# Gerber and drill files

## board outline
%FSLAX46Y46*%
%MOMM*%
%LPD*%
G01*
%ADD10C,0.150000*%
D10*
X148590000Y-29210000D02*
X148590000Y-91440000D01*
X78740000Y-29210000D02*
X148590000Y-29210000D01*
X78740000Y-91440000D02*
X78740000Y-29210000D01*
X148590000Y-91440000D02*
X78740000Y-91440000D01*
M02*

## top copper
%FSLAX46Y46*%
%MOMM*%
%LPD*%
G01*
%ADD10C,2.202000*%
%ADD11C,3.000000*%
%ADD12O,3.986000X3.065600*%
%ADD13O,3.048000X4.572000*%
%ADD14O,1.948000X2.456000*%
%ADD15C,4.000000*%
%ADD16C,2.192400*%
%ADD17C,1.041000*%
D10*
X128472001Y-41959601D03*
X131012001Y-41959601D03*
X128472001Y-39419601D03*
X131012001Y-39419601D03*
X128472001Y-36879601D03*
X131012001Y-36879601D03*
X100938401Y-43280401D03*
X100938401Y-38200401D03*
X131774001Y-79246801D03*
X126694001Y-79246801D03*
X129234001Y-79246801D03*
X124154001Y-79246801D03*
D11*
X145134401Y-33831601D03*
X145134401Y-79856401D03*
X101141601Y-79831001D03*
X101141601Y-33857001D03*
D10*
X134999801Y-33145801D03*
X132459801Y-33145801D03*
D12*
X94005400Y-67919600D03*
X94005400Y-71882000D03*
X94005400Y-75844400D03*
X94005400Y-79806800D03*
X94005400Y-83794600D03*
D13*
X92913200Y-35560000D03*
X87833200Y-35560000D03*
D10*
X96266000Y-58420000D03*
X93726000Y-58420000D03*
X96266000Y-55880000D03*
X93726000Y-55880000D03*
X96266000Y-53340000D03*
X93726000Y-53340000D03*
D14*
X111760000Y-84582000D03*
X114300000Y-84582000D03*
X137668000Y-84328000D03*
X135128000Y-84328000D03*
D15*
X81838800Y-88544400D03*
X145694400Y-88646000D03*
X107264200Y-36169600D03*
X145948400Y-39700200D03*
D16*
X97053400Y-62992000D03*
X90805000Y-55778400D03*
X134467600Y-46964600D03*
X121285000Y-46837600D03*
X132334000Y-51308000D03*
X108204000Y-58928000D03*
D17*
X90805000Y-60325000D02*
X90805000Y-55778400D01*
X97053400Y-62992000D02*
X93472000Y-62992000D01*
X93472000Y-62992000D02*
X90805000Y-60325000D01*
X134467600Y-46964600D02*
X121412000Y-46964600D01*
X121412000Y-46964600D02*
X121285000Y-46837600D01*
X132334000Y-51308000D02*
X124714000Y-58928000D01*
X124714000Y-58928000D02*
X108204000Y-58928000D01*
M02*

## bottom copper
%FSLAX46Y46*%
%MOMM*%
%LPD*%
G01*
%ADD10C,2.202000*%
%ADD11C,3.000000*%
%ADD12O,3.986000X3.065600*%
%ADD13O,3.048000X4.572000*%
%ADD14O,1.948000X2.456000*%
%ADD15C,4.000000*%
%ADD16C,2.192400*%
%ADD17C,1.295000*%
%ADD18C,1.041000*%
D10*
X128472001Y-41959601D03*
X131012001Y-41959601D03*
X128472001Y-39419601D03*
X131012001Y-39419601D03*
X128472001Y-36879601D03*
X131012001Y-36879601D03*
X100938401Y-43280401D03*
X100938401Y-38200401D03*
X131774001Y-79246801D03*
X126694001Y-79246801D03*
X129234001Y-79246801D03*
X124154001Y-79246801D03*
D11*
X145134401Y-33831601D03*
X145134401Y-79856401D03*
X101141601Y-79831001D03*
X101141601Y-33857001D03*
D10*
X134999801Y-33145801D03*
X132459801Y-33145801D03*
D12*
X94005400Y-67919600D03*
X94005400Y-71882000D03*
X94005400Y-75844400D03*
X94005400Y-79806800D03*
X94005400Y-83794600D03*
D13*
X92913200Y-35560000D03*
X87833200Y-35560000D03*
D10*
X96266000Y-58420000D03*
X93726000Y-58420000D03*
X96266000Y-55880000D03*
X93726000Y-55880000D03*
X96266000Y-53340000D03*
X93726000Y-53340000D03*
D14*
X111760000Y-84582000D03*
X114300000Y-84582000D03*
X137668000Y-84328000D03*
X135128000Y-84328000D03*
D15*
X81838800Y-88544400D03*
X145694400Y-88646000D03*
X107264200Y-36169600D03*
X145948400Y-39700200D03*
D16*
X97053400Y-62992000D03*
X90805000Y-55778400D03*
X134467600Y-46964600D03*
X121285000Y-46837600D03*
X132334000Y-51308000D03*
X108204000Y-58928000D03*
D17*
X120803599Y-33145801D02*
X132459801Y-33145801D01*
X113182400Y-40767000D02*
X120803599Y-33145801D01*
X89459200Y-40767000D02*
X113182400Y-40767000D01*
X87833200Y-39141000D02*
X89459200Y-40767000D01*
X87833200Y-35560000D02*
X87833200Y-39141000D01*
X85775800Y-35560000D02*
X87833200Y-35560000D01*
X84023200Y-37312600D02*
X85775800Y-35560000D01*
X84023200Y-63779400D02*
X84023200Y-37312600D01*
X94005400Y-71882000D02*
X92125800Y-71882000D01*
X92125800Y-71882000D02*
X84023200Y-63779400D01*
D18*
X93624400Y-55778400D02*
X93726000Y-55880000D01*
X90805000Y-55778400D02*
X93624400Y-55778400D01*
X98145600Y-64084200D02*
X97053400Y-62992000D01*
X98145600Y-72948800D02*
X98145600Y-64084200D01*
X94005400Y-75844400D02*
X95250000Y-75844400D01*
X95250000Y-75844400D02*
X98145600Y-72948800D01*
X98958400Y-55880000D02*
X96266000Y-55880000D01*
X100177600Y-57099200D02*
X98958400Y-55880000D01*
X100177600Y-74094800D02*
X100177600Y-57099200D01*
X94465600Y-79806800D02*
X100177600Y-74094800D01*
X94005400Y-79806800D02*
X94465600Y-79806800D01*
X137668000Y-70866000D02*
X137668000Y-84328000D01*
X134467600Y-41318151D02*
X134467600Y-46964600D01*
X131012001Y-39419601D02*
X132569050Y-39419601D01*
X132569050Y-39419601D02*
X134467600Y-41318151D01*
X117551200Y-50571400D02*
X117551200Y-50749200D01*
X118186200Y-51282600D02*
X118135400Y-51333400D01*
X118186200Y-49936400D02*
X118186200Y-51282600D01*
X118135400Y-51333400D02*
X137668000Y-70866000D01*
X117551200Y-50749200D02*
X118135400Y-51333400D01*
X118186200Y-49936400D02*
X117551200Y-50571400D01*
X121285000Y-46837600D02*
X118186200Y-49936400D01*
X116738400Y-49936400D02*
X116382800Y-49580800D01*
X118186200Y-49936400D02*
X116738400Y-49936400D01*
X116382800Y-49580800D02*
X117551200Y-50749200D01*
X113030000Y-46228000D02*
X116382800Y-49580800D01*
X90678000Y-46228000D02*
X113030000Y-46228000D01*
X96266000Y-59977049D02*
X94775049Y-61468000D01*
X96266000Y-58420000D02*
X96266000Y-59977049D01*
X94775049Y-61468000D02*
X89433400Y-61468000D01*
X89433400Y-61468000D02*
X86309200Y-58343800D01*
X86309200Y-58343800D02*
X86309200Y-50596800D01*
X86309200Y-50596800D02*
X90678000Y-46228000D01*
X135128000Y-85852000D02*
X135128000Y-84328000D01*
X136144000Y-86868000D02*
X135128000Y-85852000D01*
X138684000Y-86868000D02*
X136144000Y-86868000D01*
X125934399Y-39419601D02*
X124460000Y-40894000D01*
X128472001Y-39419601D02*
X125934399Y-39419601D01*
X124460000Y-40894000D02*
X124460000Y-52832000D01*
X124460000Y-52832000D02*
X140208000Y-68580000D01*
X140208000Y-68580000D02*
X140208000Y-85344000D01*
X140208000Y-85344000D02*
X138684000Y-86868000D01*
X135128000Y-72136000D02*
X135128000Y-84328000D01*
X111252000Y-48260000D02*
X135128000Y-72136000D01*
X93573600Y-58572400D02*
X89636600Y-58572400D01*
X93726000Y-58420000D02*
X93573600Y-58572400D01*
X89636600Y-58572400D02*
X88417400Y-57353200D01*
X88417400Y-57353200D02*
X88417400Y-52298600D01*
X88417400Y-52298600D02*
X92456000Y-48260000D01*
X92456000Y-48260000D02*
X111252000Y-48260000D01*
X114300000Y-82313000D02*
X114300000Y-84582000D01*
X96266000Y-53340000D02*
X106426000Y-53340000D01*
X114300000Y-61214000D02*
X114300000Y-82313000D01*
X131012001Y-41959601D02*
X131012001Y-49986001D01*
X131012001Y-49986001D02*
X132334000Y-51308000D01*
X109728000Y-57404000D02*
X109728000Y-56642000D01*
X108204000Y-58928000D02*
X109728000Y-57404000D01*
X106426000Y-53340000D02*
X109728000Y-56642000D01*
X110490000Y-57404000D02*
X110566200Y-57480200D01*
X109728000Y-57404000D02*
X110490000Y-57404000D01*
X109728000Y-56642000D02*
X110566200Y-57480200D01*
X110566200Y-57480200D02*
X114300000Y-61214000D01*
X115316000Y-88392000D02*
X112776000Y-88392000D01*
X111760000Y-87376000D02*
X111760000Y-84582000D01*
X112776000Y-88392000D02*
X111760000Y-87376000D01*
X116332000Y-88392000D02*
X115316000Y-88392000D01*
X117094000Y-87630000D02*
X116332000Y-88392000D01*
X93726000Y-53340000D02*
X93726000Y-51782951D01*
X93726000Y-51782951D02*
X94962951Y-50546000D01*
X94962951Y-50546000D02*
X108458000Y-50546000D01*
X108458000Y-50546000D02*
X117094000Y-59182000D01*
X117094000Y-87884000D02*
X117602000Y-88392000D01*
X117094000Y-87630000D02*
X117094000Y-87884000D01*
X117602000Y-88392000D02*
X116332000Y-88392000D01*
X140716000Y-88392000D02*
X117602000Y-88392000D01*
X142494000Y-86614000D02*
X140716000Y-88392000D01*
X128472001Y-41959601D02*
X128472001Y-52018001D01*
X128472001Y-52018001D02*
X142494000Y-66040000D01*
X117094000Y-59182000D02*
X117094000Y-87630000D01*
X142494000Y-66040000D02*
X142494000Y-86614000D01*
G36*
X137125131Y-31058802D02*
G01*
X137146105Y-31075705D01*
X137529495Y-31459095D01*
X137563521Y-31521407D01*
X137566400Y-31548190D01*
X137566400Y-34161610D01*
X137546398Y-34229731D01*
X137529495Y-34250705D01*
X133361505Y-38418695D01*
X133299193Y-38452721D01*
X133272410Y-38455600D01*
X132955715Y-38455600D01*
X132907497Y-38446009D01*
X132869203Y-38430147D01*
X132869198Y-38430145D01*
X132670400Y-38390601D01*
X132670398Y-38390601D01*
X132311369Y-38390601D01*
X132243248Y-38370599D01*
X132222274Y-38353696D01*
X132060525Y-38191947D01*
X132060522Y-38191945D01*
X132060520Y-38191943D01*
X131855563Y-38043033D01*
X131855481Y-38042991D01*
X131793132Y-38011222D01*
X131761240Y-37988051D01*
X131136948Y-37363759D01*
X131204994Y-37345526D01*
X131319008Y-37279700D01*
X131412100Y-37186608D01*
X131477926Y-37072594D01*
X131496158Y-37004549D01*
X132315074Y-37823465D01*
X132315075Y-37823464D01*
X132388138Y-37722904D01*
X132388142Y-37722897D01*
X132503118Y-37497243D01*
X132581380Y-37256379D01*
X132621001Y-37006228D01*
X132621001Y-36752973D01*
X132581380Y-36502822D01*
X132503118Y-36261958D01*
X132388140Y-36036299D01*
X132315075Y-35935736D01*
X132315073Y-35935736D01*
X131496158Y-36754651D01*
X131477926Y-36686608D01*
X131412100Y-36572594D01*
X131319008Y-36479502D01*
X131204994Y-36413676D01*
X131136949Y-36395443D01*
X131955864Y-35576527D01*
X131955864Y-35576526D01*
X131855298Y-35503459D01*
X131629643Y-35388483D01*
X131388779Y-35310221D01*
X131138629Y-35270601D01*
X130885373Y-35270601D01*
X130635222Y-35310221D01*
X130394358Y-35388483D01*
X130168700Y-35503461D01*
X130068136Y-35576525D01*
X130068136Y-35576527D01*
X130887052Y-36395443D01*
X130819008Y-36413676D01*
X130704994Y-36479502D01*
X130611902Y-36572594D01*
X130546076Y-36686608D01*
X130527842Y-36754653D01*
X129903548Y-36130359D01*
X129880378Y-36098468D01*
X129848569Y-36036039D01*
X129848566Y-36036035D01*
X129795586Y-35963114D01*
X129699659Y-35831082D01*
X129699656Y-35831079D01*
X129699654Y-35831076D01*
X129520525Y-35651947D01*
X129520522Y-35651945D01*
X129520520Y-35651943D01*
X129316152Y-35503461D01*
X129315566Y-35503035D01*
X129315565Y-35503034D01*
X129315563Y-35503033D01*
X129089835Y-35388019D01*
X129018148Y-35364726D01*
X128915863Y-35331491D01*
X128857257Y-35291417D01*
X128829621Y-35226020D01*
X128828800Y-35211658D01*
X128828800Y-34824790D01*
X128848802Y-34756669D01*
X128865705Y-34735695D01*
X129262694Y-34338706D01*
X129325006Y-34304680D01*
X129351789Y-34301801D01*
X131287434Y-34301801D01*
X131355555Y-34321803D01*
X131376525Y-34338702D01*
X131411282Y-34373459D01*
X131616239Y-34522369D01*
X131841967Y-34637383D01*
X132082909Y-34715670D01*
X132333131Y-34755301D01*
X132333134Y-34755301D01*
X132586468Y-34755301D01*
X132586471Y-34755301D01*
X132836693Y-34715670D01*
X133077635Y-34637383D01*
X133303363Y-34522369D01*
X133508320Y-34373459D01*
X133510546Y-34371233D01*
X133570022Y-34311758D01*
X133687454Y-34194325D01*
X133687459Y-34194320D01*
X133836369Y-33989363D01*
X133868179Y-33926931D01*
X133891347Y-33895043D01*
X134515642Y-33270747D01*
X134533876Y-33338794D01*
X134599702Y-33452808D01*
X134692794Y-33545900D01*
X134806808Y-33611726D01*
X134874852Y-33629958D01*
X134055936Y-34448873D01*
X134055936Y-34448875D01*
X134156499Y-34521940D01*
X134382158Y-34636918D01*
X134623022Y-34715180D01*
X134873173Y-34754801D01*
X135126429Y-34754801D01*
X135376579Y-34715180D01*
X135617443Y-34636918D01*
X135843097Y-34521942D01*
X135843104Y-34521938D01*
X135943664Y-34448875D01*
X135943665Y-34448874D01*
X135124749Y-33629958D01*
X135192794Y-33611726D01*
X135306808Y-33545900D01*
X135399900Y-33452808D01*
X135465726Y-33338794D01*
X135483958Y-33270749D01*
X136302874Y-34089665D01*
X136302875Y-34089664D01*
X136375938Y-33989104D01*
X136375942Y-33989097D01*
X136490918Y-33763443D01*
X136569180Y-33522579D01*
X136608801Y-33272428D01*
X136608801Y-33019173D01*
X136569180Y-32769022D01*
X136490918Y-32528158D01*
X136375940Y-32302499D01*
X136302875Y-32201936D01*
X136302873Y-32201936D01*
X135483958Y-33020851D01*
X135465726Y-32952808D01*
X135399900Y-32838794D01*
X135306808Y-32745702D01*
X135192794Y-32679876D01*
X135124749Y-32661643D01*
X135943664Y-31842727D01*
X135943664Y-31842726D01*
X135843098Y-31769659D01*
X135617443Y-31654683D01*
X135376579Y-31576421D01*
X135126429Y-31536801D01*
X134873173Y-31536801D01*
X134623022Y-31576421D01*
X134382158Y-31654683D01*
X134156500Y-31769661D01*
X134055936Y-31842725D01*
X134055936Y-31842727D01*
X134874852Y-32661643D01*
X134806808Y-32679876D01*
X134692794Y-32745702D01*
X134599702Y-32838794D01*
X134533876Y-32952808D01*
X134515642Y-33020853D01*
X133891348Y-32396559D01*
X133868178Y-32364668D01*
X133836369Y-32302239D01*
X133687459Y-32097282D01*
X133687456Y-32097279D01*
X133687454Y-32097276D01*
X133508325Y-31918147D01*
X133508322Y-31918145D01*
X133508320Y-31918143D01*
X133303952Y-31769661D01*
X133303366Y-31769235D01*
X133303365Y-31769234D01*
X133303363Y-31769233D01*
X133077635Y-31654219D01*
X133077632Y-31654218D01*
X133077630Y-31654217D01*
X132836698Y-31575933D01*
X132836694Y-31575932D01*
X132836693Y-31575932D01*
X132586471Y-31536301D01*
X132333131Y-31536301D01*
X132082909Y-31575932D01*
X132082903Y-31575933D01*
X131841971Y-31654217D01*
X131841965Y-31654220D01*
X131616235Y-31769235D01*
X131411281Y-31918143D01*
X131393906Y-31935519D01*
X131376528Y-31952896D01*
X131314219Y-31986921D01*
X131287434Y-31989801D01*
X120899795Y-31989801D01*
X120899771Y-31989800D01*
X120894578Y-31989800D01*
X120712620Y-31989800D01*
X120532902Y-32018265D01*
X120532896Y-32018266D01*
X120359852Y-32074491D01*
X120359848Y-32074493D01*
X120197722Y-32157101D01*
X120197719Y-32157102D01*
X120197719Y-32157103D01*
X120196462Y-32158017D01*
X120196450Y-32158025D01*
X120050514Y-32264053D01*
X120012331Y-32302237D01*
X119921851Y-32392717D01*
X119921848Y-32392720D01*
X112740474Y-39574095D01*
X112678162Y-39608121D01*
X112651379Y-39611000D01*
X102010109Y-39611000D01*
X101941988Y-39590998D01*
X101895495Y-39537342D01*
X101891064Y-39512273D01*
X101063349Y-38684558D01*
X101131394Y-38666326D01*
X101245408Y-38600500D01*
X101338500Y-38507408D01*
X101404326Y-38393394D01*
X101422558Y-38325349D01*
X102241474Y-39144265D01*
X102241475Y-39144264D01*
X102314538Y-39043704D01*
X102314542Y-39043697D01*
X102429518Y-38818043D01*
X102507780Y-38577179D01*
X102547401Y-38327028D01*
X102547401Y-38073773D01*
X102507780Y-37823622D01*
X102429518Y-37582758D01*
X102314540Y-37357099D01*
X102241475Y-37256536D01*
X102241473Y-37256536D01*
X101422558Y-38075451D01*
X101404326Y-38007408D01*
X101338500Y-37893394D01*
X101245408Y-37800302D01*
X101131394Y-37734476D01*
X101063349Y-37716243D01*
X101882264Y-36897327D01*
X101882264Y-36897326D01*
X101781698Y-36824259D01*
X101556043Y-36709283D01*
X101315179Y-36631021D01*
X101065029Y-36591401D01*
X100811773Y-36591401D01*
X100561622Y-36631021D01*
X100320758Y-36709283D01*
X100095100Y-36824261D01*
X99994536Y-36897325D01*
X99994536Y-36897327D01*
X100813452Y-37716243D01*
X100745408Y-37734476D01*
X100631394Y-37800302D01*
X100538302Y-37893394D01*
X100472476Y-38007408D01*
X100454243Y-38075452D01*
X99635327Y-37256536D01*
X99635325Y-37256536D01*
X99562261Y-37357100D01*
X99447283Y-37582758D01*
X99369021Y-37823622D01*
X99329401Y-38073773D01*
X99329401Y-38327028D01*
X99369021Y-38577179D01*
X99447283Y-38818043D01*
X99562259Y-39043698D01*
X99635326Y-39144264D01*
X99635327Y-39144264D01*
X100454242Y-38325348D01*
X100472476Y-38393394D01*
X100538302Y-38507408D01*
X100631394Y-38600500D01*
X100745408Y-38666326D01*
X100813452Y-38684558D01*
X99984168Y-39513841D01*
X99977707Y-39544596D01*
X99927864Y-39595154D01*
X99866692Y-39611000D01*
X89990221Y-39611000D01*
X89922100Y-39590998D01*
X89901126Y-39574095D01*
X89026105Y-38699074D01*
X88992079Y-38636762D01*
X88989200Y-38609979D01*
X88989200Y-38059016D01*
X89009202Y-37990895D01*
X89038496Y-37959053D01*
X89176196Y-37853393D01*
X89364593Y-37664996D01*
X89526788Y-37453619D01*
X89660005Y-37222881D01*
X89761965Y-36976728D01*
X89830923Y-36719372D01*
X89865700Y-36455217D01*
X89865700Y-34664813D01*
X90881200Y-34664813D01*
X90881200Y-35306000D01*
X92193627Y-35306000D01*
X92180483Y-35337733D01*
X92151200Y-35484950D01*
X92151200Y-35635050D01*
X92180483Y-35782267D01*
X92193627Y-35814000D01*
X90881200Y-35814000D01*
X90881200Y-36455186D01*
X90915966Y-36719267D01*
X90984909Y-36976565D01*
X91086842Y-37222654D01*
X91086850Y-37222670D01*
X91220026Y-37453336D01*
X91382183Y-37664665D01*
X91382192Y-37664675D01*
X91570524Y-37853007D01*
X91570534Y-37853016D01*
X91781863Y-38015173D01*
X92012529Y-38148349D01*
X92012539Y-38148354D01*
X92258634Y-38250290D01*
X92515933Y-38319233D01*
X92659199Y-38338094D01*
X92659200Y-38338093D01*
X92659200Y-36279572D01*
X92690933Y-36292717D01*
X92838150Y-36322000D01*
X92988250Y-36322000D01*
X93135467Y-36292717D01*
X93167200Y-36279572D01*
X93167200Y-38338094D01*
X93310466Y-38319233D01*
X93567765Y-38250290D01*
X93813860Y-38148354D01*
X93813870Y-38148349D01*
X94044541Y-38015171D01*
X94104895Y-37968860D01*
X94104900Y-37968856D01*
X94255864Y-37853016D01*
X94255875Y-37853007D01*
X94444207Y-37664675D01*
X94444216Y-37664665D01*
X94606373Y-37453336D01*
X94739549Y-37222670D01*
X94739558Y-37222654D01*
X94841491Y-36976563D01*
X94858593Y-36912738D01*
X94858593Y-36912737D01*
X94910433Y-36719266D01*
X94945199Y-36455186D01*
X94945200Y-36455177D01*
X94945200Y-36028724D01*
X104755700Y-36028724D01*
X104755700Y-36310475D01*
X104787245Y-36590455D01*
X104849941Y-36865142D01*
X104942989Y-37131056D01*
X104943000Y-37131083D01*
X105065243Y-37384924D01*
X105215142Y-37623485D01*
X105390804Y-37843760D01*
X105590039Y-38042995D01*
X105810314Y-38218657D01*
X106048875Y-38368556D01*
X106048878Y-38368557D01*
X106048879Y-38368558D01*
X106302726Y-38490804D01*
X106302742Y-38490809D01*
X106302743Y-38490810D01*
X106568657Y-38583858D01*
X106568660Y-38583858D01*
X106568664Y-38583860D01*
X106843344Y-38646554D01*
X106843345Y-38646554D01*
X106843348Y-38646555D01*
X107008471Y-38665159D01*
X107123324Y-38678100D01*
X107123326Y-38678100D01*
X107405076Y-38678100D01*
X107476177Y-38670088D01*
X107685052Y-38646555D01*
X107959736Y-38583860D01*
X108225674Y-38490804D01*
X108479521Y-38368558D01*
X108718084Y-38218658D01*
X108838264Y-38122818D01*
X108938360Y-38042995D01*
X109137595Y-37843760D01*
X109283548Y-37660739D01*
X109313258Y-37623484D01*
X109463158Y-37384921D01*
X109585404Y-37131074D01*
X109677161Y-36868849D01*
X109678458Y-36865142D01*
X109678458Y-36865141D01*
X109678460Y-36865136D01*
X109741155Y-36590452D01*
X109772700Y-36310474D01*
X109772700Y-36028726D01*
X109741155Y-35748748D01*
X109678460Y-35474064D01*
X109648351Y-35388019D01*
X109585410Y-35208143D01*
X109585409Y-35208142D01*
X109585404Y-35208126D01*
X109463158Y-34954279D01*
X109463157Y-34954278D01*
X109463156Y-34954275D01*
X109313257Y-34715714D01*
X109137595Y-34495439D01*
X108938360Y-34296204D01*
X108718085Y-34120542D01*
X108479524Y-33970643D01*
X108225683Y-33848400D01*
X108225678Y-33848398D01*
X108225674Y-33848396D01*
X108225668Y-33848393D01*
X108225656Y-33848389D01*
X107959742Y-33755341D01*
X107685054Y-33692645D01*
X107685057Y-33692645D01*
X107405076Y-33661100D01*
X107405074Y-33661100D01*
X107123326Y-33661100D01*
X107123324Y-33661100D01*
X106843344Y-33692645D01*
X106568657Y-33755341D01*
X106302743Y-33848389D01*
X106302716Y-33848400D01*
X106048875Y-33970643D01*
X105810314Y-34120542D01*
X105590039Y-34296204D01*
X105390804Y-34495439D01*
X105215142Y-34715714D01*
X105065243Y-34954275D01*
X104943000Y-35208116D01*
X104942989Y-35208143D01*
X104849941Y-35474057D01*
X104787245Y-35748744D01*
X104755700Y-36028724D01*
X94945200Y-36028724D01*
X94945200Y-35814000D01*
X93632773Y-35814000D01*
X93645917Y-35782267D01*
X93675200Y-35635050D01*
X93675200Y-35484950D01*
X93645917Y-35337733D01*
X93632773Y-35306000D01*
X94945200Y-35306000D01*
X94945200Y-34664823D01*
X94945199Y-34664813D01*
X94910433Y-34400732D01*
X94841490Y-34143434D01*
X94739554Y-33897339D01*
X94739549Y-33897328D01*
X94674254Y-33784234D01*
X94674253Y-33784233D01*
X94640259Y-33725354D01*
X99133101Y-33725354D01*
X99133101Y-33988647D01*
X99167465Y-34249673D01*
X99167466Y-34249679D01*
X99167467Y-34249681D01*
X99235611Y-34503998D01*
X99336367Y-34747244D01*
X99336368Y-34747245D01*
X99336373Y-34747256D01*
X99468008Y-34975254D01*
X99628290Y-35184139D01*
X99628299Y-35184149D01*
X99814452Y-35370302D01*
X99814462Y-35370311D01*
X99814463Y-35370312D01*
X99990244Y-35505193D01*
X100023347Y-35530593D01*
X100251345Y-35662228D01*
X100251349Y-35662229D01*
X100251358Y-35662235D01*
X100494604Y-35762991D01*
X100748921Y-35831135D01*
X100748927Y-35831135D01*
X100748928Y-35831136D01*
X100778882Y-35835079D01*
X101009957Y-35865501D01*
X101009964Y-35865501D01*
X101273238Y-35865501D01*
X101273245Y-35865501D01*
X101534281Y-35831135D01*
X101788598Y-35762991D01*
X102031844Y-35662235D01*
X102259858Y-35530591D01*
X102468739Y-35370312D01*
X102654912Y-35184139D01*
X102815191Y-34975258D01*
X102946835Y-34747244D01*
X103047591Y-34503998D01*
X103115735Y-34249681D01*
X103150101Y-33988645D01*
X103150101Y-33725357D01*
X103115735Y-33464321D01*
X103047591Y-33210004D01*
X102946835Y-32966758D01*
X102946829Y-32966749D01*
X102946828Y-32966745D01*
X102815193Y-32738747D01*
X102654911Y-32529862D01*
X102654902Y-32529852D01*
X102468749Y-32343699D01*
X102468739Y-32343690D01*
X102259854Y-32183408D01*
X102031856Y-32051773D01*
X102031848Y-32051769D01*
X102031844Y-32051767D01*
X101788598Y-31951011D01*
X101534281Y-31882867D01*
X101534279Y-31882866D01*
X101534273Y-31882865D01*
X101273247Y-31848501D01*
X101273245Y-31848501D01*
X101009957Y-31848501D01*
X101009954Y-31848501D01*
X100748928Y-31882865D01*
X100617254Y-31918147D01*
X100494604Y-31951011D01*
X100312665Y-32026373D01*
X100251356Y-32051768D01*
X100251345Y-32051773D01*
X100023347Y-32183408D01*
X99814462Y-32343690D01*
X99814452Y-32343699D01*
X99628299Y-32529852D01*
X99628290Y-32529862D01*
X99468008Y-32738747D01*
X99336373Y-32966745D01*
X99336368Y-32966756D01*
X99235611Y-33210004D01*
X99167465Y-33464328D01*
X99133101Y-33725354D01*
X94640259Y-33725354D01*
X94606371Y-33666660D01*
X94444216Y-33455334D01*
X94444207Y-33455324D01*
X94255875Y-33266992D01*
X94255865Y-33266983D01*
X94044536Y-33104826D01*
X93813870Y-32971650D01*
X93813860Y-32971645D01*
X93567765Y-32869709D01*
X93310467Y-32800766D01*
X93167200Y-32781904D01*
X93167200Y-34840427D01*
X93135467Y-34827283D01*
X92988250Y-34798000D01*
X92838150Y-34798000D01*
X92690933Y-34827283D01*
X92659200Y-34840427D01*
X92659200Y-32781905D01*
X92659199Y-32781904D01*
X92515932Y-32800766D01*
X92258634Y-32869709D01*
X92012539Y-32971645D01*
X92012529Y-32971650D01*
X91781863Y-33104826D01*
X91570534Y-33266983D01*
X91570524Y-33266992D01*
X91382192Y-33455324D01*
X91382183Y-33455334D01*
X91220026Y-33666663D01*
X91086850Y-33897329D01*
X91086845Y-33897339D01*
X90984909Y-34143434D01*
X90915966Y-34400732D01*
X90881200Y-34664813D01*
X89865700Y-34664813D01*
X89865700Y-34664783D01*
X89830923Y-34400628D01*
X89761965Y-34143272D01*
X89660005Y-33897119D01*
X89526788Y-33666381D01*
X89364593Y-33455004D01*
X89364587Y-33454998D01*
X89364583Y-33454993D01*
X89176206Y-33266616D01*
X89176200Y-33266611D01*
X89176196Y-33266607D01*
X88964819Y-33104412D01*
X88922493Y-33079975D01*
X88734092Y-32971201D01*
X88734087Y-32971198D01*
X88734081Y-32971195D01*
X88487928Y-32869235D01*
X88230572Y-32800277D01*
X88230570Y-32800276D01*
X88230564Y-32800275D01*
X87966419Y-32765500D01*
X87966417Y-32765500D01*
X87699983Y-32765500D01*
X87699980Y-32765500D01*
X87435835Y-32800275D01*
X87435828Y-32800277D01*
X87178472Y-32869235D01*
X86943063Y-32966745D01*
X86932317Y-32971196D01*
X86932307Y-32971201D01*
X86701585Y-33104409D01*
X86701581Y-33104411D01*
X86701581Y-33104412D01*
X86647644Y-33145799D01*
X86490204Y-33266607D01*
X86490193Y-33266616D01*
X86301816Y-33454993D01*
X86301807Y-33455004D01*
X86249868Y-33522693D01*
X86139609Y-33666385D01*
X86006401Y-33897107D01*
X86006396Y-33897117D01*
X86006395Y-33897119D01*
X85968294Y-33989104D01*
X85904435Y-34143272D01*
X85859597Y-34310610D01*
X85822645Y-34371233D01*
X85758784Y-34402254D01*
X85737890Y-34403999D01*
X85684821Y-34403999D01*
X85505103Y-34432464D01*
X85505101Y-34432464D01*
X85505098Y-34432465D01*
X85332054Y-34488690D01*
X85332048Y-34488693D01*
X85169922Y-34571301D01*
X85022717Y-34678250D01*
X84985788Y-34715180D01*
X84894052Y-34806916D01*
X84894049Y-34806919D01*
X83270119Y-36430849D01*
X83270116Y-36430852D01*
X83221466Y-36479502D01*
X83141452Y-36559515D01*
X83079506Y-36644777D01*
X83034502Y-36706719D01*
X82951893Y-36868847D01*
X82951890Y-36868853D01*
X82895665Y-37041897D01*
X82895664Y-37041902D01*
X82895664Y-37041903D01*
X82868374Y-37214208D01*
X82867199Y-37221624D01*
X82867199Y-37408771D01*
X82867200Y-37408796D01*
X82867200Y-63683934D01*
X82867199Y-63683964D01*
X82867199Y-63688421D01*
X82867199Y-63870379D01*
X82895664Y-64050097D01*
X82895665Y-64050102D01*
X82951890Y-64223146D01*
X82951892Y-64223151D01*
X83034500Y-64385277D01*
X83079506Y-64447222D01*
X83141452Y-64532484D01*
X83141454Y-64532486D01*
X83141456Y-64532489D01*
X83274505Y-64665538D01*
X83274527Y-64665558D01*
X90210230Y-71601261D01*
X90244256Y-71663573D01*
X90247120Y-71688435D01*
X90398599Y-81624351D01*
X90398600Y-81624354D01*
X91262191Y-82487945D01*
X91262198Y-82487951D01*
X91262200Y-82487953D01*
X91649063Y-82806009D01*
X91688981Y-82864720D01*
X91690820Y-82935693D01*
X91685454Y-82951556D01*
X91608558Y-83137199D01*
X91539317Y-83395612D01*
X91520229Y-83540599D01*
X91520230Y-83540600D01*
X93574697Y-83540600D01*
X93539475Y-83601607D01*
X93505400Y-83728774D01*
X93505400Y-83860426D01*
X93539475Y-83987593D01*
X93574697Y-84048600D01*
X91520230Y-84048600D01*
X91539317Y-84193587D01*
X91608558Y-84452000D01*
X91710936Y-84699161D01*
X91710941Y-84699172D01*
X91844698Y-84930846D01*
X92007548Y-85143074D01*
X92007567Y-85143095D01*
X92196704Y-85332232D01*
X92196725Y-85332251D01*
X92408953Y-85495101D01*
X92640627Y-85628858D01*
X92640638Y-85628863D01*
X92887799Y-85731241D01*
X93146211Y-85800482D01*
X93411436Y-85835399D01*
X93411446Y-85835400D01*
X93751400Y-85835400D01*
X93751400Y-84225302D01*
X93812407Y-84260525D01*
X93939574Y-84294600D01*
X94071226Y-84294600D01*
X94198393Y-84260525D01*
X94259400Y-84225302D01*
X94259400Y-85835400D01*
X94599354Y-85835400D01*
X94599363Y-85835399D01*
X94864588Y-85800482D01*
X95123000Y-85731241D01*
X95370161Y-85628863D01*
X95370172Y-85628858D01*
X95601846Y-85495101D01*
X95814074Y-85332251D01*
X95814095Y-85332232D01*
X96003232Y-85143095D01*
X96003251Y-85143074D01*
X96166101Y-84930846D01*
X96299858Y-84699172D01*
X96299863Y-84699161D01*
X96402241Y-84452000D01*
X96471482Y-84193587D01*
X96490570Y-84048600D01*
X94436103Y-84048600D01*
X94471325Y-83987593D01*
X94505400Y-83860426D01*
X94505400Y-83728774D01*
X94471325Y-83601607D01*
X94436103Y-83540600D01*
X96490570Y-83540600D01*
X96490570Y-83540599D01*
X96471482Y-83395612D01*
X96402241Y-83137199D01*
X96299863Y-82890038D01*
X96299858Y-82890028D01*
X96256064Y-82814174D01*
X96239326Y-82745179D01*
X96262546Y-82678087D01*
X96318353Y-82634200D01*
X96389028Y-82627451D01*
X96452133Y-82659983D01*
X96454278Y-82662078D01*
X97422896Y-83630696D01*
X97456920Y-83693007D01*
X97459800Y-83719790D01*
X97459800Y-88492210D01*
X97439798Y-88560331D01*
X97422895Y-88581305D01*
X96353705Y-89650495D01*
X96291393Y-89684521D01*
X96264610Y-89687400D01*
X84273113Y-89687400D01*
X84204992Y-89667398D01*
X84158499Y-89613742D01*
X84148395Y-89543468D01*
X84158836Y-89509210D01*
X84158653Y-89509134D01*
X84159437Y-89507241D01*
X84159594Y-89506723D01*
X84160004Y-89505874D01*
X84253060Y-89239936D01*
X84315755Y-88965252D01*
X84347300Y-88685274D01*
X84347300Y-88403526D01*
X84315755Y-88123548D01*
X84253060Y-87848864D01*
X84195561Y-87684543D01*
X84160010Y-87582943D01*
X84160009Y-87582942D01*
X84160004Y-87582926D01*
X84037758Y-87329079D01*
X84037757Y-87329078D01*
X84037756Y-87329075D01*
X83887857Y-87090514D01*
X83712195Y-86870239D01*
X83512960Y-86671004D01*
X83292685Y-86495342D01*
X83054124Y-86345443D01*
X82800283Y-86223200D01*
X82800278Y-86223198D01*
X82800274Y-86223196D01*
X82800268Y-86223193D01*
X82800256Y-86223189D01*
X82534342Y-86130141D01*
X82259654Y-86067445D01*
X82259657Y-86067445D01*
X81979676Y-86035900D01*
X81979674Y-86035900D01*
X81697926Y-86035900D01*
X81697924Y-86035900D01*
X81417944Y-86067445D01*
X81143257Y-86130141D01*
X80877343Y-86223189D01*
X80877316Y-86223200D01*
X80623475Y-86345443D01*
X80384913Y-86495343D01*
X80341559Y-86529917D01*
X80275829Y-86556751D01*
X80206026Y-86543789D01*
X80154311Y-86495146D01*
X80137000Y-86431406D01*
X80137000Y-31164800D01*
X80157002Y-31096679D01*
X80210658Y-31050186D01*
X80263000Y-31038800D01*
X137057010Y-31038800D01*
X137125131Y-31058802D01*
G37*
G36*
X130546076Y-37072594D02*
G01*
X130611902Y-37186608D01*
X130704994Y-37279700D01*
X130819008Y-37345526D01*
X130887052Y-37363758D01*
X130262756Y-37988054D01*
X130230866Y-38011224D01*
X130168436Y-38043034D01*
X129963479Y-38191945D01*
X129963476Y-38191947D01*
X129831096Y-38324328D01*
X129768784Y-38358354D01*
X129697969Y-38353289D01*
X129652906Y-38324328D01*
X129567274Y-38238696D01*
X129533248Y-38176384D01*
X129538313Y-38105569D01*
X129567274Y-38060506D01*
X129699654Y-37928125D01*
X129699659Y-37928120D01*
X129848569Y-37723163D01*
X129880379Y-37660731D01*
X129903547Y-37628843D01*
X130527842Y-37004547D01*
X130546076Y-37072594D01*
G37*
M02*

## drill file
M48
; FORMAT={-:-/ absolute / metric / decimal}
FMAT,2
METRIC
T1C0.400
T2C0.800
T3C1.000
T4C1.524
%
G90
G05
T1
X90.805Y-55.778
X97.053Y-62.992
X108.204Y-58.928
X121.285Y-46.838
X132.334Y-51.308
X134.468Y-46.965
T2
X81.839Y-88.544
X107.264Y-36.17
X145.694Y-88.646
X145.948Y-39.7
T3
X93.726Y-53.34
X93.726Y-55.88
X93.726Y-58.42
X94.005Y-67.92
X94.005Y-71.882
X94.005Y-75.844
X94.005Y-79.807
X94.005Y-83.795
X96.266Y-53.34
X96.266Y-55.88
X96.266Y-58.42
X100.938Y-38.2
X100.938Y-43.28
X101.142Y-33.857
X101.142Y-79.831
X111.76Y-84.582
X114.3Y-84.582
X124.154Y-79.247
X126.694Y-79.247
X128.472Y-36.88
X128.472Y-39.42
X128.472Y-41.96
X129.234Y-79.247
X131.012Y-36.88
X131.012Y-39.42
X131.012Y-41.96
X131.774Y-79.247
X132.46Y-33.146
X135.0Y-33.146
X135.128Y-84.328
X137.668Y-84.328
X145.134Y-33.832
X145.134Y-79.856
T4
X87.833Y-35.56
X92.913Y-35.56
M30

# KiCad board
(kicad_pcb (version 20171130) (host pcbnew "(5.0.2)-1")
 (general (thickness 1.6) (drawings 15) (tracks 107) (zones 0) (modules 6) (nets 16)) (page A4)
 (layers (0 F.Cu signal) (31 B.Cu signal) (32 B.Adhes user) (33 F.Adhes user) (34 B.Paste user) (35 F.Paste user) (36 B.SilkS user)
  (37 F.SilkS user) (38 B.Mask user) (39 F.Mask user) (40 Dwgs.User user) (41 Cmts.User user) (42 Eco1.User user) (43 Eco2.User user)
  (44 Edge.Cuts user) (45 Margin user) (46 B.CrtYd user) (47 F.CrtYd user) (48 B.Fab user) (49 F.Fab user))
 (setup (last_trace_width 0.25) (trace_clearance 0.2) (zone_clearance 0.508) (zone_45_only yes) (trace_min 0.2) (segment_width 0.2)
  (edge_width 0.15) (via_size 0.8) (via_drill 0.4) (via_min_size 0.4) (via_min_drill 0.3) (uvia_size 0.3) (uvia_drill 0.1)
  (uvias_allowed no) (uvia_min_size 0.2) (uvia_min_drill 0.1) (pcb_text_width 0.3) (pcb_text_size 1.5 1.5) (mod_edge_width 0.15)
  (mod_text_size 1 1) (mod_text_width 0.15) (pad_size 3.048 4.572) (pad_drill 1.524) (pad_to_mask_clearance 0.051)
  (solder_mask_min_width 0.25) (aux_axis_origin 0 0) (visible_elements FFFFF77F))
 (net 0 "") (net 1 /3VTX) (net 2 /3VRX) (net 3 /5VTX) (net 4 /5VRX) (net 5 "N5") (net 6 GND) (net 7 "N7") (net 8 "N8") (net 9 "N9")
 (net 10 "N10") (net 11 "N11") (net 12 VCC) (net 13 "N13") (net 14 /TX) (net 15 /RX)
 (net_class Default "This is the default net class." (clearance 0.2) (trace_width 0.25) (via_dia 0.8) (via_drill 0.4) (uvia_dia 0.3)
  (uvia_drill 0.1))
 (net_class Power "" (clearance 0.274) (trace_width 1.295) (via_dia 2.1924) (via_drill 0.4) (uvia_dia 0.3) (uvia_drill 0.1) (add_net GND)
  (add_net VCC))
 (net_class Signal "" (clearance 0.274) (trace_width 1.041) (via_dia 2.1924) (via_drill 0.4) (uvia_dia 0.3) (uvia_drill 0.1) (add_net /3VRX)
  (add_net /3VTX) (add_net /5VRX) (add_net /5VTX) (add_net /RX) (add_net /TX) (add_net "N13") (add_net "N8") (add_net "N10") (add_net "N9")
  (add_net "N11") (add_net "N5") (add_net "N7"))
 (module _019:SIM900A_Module (layer F.Cu) (at 123.138001 56.844001)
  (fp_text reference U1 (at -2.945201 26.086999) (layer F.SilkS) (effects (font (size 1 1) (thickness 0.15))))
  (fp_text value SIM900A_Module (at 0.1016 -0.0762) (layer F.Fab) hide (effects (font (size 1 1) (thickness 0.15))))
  (pad 6 thru_hole circle (at 5.334 -14.8844) (size 2.202 2.202) (drill 1) (layers *.Cu *.Mask) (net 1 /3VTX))
  (pad 5 thru_hole circle (at 7.874 -14.8844) (size 2.202 2.202) (drill 1) (layers *.Cu *.Mask) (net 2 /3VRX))
  (pad 4 thru_hole circle (at 5.334 -17.4244) (size 2.202 2.202) (drill 1) (layers *.Cu *.Mask) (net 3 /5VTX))
  (pad 3 thru_hole circle (at 7.874 -17.4244) (size 2.202 2.202) (drill 1) (layers *.Cu *.Mask) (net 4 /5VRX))
  (pad 2 thru_hole circle (at 5.334 -19.9644) (size 2.202 2.202) (drill 1) (layers *.Cu *.Mask) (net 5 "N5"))
  (pad 1 thru_hole circle (at 7.874 -19.9644) (size 2.202 2.202) (drill 1) (layers *.Cu *.Mask) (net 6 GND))
  (pad 9 thru_hole circle (at -22.1996 -13.5636) (size 2.202 2.202) (drill 1) (layers *.Cu *.Mask) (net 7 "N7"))
  (pad 7 thru_hole circle (at -22.1996 -18.6436) (size 2.202 2.202) (drill 1) (layers *.Cu *.Mask) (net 6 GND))
  (pad 10 thru_hole circle (at 8.636 22.4028) (size 2.202 2.202) (drill 1) (layers *.Cu *.Mask) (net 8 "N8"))
  (pad 12 thru_hole circle (at 3.556 22.4028) (size 2.202 2.202) (drill 1) (layers *.Cu *.Mask) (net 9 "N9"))
  (pad 11 thru_hole circle (at 6.096 22.4028) (size 2.202 2.202) (drill 1) (layers *.Cu *.Mask) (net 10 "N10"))
  (pad 13 thru_hole circle (at 1.016 22.4028) (size 2.202 2.202) (drill 1) (layers *.Cu *.Mask) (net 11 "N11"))
  (pad "" thru_hole circle (at 21.9964 -23.0124) (size 3 3) (drill 1) (layers *.Cu *.Mask))
  (pad "" thru_hole circle (at 21.9964 23.0124) (size 3 3) (drill 1) (layers *.Cu *.Mask))
  (pad "" thru_hole circle (at -21.9964 22.987) (size 3 3) (drill 1) (layers *.Cu *.Mask))
  (pad "" thru_hole circle (at -21.9964 -22.987) (size 3 3) (drill 1) (layers *.Cu *.Mask))
  (pad 14 thru_hole circle (at 11.8618 -23.6982) (size 2.202 2.202) (drill 1) (layers *.Cu *.Mask) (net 6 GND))
  (pad 15 thru_hole circle (at 9.3218 -23.6982) (size 2.202 2.202) (drill 1) (layers *.Cu *.Mask) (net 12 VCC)))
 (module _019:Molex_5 (layer F.Cu) (at 94.0054 83.7946)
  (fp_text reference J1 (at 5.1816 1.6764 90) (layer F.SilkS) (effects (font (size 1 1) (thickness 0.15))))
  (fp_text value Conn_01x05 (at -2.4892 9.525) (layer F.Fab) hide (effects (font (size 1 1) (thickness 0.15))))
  (pad 5 thru_hole oval (at 0 -15.875) (size 3.986 3.0656) (drill 1) (layers *.Cu *.Mask) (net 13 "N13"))
  (pad 4 thru_hole oval (at 0 -11.9126) (size 3.986 3.0656) (drill 1) (layers *.Cu *.Mask) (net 12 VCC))
  (pad 3 thru_hole oval (at 0 -7.9502) (size 3.986 3.0656) (drill 1) (layers *.Cu *.Mask) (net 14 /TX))
  (pad 2 thru_hole oval (at 0 -3.9878) (size 3.986 3.0656) (drill 1) (layers *.Cu *.Mask) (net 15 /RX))
  (pad 1 thru_hole oval (at 0 0) (size 3.986 3.0656) (drill 1) (layers *.Cu *.Mask) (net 6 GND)))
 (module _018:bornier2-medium (layer F.Cu) (at 90.3732 35.56 180)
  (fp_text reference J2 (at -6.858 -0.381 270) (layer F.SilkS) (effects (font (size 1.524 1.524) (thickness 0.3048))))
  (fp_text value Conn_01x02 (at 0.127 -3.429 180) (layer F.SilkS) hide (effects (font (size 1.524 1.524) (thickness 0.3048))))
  (pad 1 thru_hole oval (at -2.54 0 180) (size 3.048 4.572) (drill 1.524) (layers *.Cu *.Mask F.SilkS) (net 6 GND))
  (pad 2 thru_hole oval (at 2.54 0 180) (size 3.048 4.572) (drill 1.524) (layers *.Cu *.Mask F.SilkS) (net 12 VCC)))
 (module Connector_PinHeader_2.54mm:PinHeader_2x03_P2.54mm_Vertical (layer F.Cu) (at 96.266 58.42 180)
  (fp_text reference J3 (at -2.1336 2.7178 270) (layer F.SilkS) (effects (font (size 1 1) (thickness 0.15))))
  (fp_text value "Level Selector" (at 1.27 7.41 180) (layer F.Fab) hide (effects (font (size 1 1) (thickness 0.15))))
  (pad 1 thru_hole circle (at 0 0 180) (size 2.202 2.202) (drill 1) (layers *.Cu *.Mask) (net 4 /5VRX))
  (pad 2 thru_hole circle (at 2.54 0 180) (size 2.202 2.202) (drill 1) (layers *.Cu *.Mask) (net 3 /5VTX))
  (pad 3 thru_hole circle (at 0 2.54 180) (size 2.202 2.202) (drill 1) (layers *.Cu *.Mask) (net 15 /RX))
  (pad 4 thru_hole circle (at 2.54 2.54 180) (size 2.202 2.202) (drill 1) (layers *.Cu *.Mask) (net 14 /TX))
  (pad 5 thru_hole circle (at 0 5.08 180) (size 2.202 2.202) (drill 1) (layers *.Cu *.Mask) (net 2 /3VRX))
  (pad 6 thru_hole circle (at 2.54 5.08 180) (size 2.202 2.202) (drill 1) (layers *.Cu *.Mask) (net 1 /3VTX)))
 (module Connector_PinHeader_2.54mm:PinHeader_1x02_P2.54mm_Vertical (layer F.Cu) (at 111.76 84.582 90)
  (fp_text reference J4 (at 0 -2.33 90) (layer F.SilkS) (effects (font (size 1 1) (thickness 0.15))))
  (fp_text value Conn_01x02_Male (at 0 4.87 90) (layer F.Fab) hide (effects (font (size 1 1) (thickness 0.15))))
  (pad 1 thru_hole oval (at 0 0 90) (size 2.456 1.948) (drill 1) (layers *.Cu *.Mask) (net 1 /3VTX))
  (pad 2 thru_hole oval (at 0 2.54 90) (size 2.456 1.948) (drill 1) (layers *.Cu *.Mask) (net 2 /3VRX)))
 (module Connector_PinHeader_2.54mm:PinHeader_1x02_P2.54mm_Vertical (layer F.Cu) (at 135.128 84.328 90)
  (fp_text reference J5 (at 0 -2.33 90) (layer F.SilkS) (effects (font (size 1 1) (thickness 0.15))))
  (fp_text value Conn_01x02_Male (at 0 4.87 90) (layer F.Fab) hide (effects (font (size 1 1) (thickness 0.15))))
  (pad 2 thru_hole oval (at 0 2.54 90) (size 2.456 1.948) (drill 1) (layers *.Cu *.Mask) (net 4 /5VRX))
  (pad 1 thru_hole oval (at 0 0 90) (size 2.456 1.948) (drill 1) (layers *.Cu *.Mask) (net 3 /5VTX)))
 (gr_line (start 148.59 29.21) (end 148.59 91.44) (layer Edge.Cuts) (width 0.15))
 (gr_line (start 78.74 29.21) (end 148.59 29.21) (layer Edge.Cuts) (width 0.15))
 (gr_line (start 78.74 91.44) (end 78.74 29.21) (layer Edge.Cuts) (width 0.15))
 (gr_line (start 148.59 91.44) (end 78.74 91.44) (layer Edge.Cuts) (width 0.15))
 (via (at 81.8388 88.5444) (size 4) (drill 0.8) (layers F.Cu B.Cu) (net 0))
 (via (at 145.6944 88.646) (size 4) (drill 0.8) (layers F.Cu B.Cu) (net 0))
 (via (at 107.2642 36.1696) (size 4) (drill 0.8) (layers F.Cu B.Cu) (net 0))
 (via (at 145.9484 39.7002) (size 4) (drill 0.8) (layers F.Cu B.Cu) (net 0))
 (segment (start 120.803599 33.145801) (end 132.459801 33.145801) (width 1.295) (layer B.Cu) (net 12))
 (segment (start 113.1824 40.767) (end 120.803599 33.145801) (width 1.295) (layer B.Cu) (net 12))
 (segment (start 89.4592 40.767) (end 113.1824 40.767) (width 1.295) (layer B.Cu) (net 12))
 (segment (start 87.8332 39.141) (end 89.4592 40.767) (width 1.295) (layer B.Cu) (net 12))
 (segment (start 87.8332 35.56) (end 87.8332 39.141) (width 1.295) (layer B.Cu) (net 12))
 (segment (start 85.7758 35.56) (end 87.8332 35.56) (width 1.295) (layer B.Cu) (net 12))
 (segment (start 84.0232 37.3126) (end 85.7758 35.56) (width 1.295) (layer B.Cu) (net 12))
 (segment (start 84.0232 63.7794) (end 84.0232 37.3126) (width 1.295) (layer B.Cu) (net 12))
 (segment (start 94.0054 71.882) (end 92.1258 71.882) (width 1.295) (layer B.Cu) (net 12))
 (segment (start 92.1258 71.882) (end 84.0232 63.7794) (width 1.295) (layer B.Cu) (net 12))
 (via (at 97.0534 62.992) (size 2.1924) (drill 0.4) (layers F.Cu B.Cu) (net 14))
 (via (at 90.805 55.7784) (size 2.1924) (drill 0.4) (layers F.Cu B.Cu) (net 14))
 (segment (start 93.6244 55.7784) (end 93.726 55.88) (width 1.041) (layer B.Cu) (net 14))
 (segment (start 90.805 55.7784) (end 93.6244 55.7784) (width 1.041) (layer B.Cu) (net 14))
 (segment (start 90.805 60.325) (end 90.805 55.7784) (width 1.041) (layer F.Cu) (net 14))
 (segment (start 97.0534 62.992) (end 93.472 62.992) (width 1.041) (layer F.Cu) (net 14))
 (segment (start 93.472 62.992) (end 90.805 60.325) (width 1.041) (layer F.Cu) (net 14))
 (segment (start 98.1456 64.0842) (end 97.0534 62.992) (width 1.041) (layer B.Cu) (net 14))
 (segment (start 98.1456 72.9488) (end 98.1456 64.0842) (width 1.041) (layer B.Cu) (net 14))
 (segment (start 94.0054 75.8444) (end 95.25 75.8444) (width 1.041) (layer B.Cu) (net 14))
 (segment (start 95.25 75.8444) (end 98.1456 72.9488) (width 1.041) (layer B.Cu) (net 14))
 (segment (start 98.9584 55.88) (end 96.266 55.88) (width 1.041) (layer B.Cu) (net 15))
 (segment (start 100.1776 57.0992) (end 98.9584 55.88) (width 1.041) (layer B.Cu) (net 15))
 (segment (start 100.1776 74.0948) (end 100.1776 57.0992) (width 1.041) (layer B.Cu) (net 15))
 (segment (start 94.4656 79.8068) (end 100.1776 74.0948) (width 1.041) (layer B.Cu) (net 15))
 (segment (start 94.0054 79.8068) (end 94.4656 79.8068) (width 1.041) (layer B.Cu) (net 15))
 (segment (start 137.668 70.866) (end 137.668 84.328) (width 1.041) (layer B.Cu) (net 4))
 (via (at 134.4676 46.9646) (size 2.1924) (drill 0.4) (layers F.Cu B.Cu) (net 4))
 (segment (start 134.4676 41.318151) (end 134.4676 46.9646) (width 1.041) (layer B.Cu) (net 4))
 (segment (start 131.012001 39.419601) (end 132.56905 39.419601) (width 1.041) (layer B.Cu) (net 4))
 (segment (start 132.56905 39.419601) (end 134.4676 41.318151) (width 1.041) (layer B.Cu) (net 4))
 (via (at 121.285 46.8376) (size 2.1924) (drill 0.4) (layers F.Cu B.Cu) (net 4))
 (segment (start 134.4676 46.9646) (end 121.412 46.9646) (width 1.041) (layer F.Cu) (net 4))
 (segment (start 121.412 46.9646) (end 121.285 46.8376) (width 1.041) (layer F.Cu) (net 4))
 (segment (start 117.5512 50.5714) (end 117.5512 50.7492) (width 1.041) (layer B.Cu) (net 4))
 (segment (start 118.1862 51.2826) (end 118.1354 51.3334) (width 1.041) (layer B.Cu) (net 4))
 (segment (start 118.1862 49.9364) (end 118.1862 51.2826) (width 1.041) (layer B.Cu) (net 4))
 (segment (start 118.1354 51.3334) (end 137.668 70.866) (width 1.041) (layer B.Cu) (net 4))
 (segment (start 117.5512 50.7492) (end 118.1354 51.3334) (width 1.041) (layer B.Cu) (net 4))
 (segment (start 118.1862 49.9364) (end 117.5512 50.5714) (width 1.041) (layer B.Cu) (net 4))
 (segment (start 121.285 46.8376) (end 118.1862 49.9364) (width 1.041) (layer B.Cu) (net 4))
 (segment (start 116.7384 49.9364) (end 116.3828 49.5808) (width 1.041) (layer B.Cu) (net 4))
 (segment (start 118.1862 49.9364) (end 116.7384 49.9364) (width 1.041) (layer B.Cu) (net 4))
 (segment (start 116.3828 49.5808) (end 117.5512 50.7492) (width 1.041) (layer B.Cu) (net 4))
 (segment (start 113.03 46.228) (end 116.3828 49.5808) (width 1.041) (layer B.Cu) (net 4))
 (segment (start 90.678 46.228) (end 113.03 46.228) (width 1.041) (layer B.Cu) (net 4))
 (segment (start 96.266 59.977049) (end 94.775049 61.468) (width 1.041) (layer B.Cu) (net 4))
 (segment (start 96.266 58.42) (end 96.266 59.977049) (width 1.041) (layer B.Cu) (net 4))
 (segment (start 94.775049 61.468) (end 89.4334 61.468) (width 1.041) (layer B.Cu) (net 4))
 (segment (start 89.4334 61.468) (end 86.3092 58.3438) (width 1.041) (layer B.Cu) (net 4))
 (segment (start 86.3092 58.3438) (end 86.3092 50.5968) (width 1.041) (layer B.Cu) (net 4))
 (segment (start 86.3092 50.5968) (end 90.678 46.228) (width 1.041) (layer B.Cu) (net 4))
 (segment (start 135.128 85.852) (end 135.128 84.328) (width 1.041) (layer B.Cu) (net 3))
 (segment (start 136.144 86.868) (end 135.128 85.852) (width 1.041) (layer B.Cu) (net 3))
 (segment (start 138.684 86.868) (end 136.144 86.868) (width 1.041) (layer B.Cu) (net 3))
 (segment (start 125.934399 39.419601) (end 124.46 40.894) (width 1.041) (layer B.Cu) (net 3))
 (segment (start 128.472001 39.419601) (end 125.934399 39.419601) (width 1.041) (layer B.Cu) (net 3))
 (segment (start 124.46 40.894) (end 124.46 52.832) (width 1.041) (layer B.Cu) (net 3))
 (segment (start 124.46 52.832) (end 140.208 68.58) (width 1.041) (layer B.Cu) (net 3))
 (segment (start 140.208 68.58) (end 140.208 85.344) (width 1.041) (layer B.Cu) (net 3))
 (segment (start 140.208 85.344) (end 138.684 86.868) (width 1.041) (layer B.Cu) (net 3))
 (segment (start 135.128 72.136) (end 135.128 84.328) (width 1.041) (layer B.Cu) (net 3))
 (segment (start 111.252 48.26) (end 135.128 72.136) (width 1.041) (layer B.Cu) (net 3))
 (segment (start 93.5736 58.5724) (end 89.6366 58.5724) (width 1.041) (layer B.Cu) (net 3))
 (segment (start 93.726 58.42) (end 93.5736 58.5724) (width 1.041) (layer B.Cu) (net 3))
 (segment (start 89.6366 58.5724) (end 88.4174 57.3532) (width 1.041) (layer B.Cu) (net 3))
 (segment (start 88.4174 57.3532) (end 88.4174 52.2986) (width 1.041) (layer B.Cu) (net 3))
 (segment (start 88.4174 52.2986) (end 92.456 48.26) (width 1.041) (layer B.Cu) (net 3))
 (segment (start 92.456 48.26) (end 111.252 48.26) (width 1.041) (layer B.Cu) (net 3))
 (segment (start 114.3 82.313) (end 114.3 84.582) (width 1.041) (layer B.Cu) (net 2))
 (segment (start 96.266 53.34) (end 106.426 53.34) (width 1.041) (layer B.Cu) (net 2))
 (segment (start 114.3 61.214) (end 114.3 82.313) (width 1.041) (layer B.Cu) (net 2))
 (via (at 132.334 51.308) (size 2.1924) (drill 0.4) (layers F.Cu B.Cu) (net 2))
 (segment (start 131.012001 41.959601) (end 131.012001 49.986001) (width 1.041) (layer B.Cu) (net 2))
 (segment (start 131.012001 49.986001) (end 132.334 51.308) (width 1.041) (layer B.Cu) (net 2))
 (via (at 108.204 58.928) (size 2.1924) (drill 0.4) (layers F.Cu B.Cu) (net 2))
 (segment (start 132.334 51.308) (end 124.714 58.928) (width 1.041) (layer F.Cu) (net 2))
 (segment (start 124.714 58.928) (end 108.204 58.928) (width 1.041) (layer F.Cu) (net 2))
 (segment (start 109.728 57.404) (end 109.728 56.642) (width 1.041) (layer B.Cu) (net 2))
 (segment (start 108.204 58.928) (end 109.728 57.404) (width 1.041) (layer B.Cu) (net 2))
 (segment (start 106.426 53.34) (end 109.728 56.642) (width 1.041) (layer B.Cu) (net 2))
 (segment (start 110.49 57.404) (end 110.5662 57.4802) (width 1.041) (layer B.Cu) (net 2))
 (segment (start 109.728 57.404) (end 110.49 57.404) (width 1.041) (layer B.Cu) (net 2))
 (segment (start 109.728 56.642) (end 110.5662 57.4802) (width 1.041) (layer B.Cu) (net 2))
 (segment (start 110.5662 57.4802) (end 114.3 61.214) (width 1.041) (layer B.Cu) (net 2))
 (segment (start 115.316 88.392) (end 112.776 88.392) (width 1.041) (layer B.Cu) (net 1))
 (segment (start 111.76 87.376) (end 111.76 84.582) (width 1.041) (layer B.Cu) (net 1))
 (segment (start 112.776 88.392) (end 111.76 87.376) (width 1.041) (layer B.Cu) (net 1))
 (segment (start 116.332 88.392) (end 115.316 88.392) (width 1.041) (layer B.Cu) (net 1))
 (segment (start 117.094 87.63) (end 116.332 88.392) (width 1.041) (layer B.Cu) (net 1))
 (segment (start 93.726 53.34) (end 93.726 51.782951) (width 1.041) (layer B.Cu) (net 1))
 (segment (start 93.726 51.782951) (end 94.962951 50.546) (width 1.041) (layer B.Cu) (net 1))
 (segment (start 94.962951 50.546) (end 108.458 50.546) (width 1.041) (layer B.Cu) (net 1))
 (segment (start 108.458 50.546) (end 117.094 59.182) (width 1.041) (layer B.Cu) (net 1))
 (segment (start 117.094 87.884) (end 117.602 88.392) (width 1.041) (layer B.Cu) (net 1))
 (segment (start 117.094 87.63) (end 117.094 87.884) (width 1.041) (layer B.Cu) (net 1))
 (segment (start 117.602 88.392) (end 116.332 88.392) (width 1.041) (layer B.Cu) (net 1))
 (segment (start 140.716 88.392) (end 117.602 88.392) (width 1.041) (layer B.Cu) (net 1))
 (segment (start 142.494 86.614) (end 140.716 88.392) (width 1.041) (layer B.Cu) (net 1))
 (segment (start 128.472001 41.959601) (end 128.472001 52.018001) (width 1.041) (layer B.Cu) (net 1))
 (segment (start 128.472001 52.018001) (end 142.494 66.04) (width 1.041) (layer B.Cu) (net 1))
 (segment (start 117.094 59.182) (end 117.094 87.63) (width 1.041) (layer B.Cu) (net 1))
 (segment (start 142.494 66.04) (end 142.494 86.614) (width 1.041) (layer B.Cu) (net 1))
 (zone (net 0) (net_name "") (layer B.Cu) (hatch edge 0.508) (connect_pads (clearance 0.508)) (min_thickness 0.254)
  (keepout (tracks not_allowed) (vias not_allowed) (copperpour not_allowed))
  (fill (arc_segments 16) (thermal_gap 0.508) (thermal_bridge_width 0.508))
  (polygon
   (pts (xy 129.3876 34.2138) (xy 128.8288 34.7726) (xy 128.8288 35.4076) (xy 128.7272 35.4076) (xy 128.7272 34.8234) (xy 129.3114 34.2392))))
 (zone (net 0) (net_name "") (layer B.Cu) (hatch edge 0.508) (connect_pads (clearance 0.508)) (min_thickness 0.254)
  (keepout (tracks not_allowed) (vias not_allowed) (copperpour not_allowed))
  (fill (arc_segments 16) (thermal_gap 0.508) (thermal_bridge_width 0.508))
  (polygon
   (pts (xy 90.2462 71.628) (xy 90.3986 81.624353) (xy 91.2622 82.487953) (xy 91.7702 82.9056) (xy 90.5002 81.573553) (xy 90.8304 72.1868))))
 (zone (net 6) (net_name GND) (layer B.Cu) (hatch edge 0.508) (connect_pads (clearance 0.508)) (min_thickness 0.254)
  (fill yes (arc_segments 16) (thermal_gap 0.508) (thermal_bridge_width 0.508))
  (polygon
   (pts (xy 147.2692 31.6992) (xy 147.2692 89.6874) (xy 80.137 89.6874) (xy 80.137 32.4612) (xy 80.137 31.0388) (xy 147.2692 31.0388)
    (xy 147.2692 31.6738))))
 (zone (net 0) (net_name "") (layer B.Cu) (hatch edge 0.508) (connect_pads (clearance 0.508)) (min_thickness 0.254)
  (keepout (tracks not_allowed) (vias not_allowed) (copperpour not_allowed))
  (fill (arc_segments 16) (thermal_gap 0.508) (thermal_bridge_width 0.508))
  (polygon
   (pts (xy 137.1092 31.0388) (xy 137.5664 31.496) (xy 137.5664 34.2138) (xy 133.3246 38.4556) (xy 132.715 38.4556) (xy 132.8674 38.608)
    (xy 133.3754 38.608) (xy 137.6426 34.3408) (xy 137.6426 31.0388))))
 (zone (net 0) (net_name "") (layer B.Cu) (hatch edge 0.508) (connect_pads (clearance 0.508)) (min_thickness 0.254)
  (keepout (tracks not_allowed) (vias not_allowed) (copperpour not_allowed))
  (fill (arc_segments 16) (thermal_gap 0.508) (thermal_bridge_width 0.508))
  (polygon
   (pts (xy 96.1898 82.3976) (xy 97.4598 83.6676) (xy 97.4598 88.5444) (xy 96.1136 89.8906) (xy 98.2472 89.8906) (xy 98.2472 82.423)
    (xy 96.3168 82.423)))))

